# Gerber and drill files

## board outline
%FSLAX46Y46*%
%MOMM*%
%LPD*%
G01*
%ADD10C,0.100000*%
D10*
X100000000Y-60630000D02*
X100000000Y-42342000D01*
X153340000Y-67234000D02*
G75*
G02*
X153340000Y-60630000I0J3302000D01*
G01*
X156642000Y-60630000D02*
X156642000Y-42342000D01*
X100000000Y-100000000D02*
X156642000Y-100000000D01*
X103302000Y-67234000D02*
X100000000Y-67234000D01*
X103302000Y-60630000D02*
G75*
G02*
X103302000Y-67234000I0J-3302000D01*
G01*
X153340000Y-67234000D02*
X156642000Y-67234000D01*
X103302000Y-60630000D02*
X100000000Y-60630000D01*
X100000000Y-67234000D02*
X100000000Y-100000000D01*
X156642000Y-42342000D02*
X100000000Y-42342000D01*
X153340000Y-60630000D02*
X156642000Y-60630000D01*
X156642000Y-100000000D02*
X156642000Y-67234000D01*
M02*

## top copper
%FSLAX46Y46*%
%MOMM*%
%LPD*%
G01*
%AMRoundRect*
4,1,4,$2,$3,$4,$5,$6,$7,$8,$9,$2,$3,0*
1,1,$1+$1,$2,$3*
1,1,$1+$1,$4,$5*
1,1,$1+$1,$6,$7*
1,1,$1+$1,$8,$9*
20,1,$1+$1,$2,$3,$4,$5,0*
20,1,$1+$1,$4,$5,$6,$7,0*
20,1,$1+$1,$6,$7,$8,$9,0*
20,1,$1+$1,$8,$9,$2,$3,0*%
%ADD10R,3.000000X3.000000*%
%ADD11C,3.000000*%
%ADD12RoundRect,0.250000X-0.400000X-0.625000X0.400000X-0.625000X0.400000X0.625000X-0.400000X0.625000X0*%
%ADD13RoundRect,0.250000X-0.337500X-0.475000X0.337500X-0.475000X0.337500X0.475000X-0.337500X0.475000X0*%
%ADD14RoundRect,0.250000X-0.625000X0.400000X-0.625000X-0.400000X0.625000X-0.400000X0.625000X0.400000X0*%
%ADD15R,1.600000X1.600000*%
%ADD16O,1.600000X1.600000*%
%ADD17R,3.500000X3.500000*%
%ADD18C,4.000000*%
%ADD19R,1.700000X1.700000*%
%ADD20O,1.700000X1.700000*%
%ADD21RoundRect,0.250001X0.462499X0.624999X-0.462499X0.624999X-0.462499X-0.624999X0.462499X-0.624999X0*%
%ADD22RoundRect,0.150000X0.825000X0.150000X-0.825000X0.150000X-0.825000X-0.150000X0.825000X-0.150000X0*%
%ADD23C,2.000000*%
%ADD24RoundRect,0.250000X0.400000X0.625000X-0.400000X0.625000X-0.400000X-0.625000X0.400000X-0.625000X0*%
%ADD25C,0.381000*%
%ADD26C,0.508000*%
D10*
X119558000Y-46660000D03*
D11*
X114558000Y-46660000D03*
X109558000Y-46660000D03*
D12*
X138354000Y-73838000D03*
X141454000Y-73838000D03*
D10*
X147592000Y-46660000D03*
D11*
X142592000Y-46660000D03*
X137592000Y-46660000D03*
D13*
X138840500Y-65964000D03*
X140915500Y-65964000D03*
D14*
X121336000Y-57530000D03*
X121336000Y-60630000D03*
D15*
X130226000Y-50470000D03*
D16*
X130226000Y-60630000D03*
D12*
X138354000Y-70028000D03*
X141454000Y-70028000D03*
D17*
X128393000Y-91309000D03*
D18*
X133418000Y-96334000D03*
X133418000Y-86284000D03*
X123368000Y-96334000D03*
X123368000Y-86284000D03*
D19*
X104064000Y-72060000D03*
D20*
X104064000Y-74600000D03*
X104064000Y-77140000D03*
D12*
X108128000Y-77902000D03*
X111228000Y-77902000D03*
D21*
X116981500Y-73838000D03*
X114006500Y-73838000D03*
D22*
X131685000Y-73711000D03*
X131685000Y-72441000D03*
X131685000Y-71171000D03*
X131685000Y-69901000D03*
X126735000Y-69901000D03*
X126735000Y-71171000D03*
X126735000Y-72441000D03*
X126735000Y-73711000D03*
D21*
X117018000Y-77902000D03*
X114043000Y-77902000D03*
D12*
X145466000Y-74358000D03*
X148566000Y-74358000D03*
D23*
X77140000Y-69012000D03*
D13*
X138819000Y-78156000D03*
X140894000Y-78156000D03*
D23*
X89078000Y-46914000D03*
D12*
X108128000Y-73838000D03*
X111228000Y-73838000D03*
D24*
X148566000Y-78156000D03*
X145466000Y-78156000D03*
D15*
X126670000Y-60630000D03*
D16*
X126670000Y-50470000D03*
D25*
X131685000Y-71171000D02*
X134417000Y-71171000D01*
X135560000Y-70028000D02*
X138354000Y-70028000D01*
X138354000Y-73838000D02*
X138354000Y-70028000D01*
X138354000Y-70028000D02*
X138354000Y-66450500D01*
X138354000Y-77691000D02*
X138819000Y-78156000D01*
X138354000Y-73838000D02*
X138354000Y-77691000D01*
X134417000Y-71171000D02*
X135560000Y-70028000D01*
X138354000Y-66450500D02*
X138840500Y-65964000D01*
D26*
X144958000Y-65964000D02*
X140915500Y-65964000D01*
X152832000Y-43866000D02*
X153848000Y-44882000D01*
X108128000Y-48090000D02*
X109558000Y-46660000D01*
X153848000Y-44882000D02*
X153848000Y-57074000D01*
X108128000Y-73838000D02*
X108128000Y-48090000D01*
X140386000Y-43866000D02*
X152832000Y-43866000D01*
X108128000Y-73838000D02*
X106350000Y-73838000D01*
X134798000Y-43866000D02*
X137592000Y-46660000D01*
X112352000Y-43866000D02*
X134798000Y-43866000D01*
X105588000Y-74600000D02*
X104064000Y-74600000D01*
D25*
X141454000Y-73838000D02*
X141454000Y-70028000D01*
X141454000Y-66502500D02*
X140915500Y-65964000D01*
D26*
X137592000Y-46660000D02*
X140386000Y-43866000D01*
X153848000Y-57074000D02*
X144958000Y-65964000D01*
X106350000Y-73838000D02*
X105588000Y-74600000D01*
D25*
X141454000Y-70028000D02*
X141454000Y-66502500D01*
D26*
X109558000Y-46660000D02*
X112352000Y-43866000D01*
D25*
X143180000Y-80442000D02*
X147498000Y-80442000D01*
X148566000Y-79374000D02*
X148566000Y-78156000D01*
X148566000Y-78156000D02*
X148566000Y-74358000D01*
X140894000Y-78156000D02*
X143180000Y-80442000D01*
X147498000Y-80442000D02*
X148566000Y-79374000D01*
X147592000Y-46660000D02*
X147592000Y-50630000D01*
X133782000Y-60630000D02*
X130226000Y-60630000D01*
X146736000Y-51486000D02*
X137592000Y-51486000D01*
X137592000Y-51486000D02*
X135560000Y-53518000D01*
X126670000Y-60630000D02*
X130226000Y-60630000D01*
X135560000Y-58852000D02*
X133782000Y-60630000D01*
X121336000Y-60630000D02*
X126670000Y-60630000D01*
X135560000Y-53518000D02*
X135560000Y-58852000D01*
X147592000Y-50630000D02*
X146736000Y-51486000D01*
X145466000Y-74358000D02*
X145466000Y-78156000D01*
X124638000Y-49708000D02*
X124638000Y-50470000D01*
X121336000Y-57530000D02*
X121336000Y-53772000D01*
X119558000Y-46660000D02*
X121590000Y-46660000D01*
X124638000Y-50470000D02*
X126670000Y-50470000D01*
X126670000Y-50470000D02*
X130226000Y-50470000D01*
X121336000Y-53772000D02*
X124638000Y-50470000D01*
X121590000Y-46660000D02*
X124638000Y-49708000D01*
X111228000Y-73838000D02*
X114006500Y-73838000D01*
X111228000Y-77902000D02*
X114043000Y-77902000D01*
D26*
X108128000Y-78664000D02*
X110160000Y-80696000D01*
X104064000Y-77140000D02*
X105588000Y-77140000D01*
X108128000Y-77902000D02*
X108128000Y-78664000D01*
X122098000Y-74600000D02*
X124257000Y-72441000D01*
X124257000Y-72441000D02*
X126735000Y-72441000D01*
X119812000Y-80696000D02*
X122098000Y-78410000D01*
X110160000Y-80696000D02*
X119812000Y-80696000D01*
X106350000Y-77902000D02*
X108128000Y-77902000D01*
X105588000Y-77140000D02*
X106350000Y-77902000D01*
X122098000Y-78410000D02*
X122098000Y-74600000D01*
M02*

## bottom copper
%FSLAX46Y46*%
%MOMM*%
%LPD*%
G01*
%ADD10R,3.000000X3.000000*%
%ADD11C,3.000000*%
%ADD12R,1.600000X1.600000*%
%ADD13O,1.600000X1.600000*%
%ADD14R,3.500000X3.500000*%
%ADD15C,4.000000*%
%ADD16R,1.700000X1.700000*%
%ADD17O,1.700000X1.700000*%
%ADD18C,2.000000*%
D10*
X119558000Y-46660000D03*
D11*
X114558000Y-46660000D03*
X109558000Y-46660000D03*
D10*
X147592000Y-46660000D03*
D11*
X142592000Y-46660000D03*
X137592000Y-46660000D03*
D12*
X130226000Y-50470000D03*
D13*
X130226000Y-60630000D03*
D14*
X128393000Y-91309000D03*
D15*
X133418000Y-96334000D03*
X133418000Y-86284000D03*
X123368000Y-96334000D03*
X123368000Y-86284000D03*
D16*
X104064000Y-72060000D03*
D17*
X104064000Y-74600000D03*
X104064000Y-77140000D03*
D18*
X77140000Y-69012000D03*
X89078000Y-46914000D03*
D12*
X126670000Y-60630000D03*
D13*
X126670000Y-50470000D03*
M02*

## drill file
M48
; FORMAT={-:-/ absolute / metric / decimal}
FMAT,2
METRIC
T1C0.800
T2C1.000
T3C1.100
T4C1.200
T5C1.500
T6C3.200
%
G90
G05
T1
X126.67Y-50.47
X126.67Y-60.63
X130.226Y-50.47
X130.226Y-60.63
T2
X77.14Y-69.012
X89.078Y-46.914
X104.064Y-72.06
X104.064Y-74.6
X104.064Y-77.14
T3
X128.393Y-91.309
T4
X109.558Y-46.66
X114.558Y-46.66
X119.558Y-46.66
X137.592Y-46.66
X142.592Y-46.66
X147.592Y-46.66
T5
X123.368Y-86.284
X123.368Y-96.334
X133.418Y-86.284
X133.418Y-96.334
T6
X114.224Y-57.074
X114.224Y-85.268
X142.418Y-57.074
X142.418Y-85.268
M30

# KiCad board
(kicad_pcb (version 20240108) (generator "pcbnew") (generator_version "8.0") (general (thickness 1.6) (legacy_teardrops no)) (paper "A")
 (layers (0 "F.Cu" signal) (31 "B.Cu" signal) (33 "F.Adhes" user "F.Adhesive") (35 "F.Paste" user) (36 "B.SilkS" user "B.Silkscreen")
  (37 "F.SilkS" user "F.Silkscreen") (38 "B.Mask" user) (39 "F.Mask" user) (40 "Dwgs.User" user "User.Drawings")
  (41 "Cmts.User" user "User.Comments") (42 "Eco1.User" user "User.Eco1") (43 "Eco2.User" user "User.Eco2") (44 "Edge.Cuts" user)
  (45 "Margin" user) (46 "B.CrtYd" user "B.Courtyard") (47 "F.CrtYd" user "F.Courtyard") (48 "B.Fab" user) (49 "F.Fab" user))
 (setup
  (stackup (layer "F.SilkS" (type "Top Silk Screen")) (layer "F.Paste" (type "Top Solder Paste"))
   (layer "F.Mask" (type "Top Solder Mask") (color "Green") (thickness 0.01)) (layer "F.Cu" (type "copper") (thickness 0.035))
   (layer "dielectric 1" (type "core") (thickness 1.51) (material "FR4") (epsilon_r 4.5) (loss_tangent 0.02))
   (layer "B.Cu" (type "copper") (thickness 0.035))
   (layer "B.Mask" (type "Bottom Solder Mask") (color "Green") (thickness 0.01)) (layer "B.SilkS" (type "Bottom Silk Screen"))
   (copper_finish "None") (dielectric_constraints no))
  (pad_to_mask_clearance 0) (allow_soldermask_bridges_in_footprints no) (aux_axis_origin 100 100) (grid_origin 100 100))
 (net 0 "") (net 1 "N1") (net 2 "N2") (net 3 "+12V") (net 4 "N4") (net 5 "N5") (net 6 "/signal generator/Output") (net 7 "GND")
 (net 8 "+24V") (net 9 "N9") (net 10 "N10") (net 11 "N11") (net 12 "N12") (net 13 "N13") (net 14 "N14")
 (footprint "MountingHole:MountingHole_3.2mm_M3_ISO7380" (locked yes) (layer "F.Cu") (at 142.418 85.268)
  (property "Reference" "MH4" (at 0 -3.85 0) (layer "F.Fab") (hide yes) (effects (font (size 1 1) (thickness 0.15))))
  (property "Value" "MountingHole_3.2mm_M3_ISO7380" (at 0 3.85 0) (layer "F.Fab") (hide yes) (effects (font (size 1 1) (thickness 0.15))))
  (pad "" np_thru_hole circle (at 0 0) (size 3.2 3.2) (drill 3.2) (layers "*.Cu" "*.Mask")))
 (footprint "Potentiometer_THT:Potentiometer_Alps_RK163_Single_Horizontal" (layer "F.Cu") (at 119.558 46.66 -90)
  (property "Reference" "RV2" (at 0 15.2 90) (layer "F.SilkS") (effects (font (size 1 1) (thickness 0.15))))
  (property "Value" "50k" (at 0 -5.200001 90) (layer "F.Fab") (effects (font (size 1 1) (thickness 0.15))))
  (pad "1" thru_hole rect (at 0 0 90) (size 3 3) (drill 1.2) (layers "*.Cu" "*.Mask") (remove_unused_layers no) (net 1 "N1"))
  (pad "2" thru_hole circle (at 0 5 90) (size 3 3) (drill 1.2) (layers "*.Cu" "*.Mask") (remove_unused_layers no) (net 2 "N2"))
  (pad "3" thru_hole circle (at 0 10 90) (size 3 3) (drill 1.2) (layers "*.Cu" "*.Mask") (remove_unused_layers no) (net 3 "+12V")))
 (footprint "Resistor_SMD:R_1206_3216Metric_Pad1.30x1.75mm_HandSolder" (layer "F.Cu") (at 139.904 73.838)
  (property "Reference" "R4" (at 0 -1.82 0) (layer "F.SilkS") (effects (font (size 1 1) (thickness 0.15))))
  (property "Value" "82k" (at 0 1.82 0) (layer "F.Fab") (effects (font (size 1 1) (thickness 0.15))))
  (pad "1" smd roundrect (at -1.55 0) (size 1.3 1.75) (layers "F.Cu" "F.Paste" "F.Mask") (roundrect_rratio 0.192308) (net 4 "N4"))
  (pad "2" smd roundrect (at 1.55 0) (size 1.3 1.75) (layers "F.Cu" "F.Paste" "F.Mask") (roundrect_rratio 0.192308) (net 3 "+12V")))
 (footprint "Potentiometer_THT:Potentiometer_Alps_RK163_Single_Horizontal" (layer "F.Cu") (at 147.592 46.66 -90)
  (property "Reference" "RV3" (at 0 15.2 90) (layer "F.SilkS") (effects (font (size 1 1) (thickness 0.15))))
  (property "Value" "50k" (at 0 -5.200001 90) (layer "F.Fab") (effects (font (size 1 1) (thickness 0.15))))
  (pad "1" thru_hole rect (at 0 0 90) (size 3 3) (drill 1.2) (layers "*.Cu" "*.Mask") (remove_unused_layers no) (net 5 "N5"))
  (pad "2" thru_hole circle (at 0 5 90) (size 3 3) (drill 1.2) (layers "*.Cu" "*.Mask") (remove_unused_layers no)
   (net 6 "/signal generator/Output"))
  (pad "3" thru_hole circle (at 0 10 90) (size 3 3) (drill 1.2) (layers "*.Cu" "*.Mask") (remove_unused_layers no) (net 3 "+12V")))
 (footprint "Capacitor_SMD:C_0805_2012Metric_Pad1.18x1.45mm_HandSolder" (layer "F.Cu") (at 139.878 65.964)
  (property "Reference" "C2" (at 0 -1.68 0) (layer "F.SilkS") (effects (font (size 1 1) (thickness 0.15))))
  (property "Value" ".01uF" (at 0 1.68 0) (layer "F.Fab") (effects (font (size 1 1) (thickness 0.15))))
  (pad "1" smd roundrect (at -1.0375 0) (size 1.175 1.45) (layers "F.Cu" "F.Paste" "F.Mask") (roundrect_rratio 0.212766) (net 4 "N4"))
  (pad "2" smd roundrect (at 1.0375 0) (size 1.175 1.45) (layers "F.Cu" "F.Paste" "F.Mask") (roundrect_rratio 0.212766) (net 3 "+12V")))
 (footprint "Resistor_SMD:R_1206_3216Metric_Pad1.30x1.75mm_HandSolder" (layer "F.Cu") (at 121.336 59.08 -90)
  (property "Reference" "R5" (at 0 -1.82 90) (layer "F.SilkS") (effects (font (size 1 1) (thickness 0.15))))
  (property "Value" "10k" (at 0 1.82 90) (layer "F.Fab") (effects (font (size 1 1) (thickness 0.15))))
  (pad "1" smd roundrect (at -1.55 0 270) (size 1.3 1.75) (layers "F.Cu" "F.Paste" "F.Mask") (roundrect_rratio 0.192308) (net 1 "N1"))
  (pad "2" smd roundrect (at 1.55 0 270) (size 1.3 1.75) (layers "F.Cu" "F.Paste" "F.Mask") (roundrect_rratio 0.192308) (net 5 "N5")))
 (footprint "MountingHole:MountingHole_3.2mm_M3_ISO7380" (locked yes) (layer "F.Cu") (at 114.224 85.268)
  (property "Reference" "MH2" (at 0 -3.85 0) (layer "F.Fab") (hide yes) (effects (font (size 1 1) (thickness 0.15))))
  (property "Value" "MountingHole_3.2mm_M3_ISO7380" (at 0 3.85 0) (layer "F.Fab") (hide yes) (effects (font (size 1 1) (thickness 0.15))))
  (pad "" np_thru_hole circle (at 0 0) (size 3.2 3.2) (drill 3.2) (layers "*.Cu" "*.Mask")))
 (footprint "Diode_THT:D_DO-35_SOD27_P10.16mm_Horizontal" (layer "F.Cu") (at 130.226 50.47 -90)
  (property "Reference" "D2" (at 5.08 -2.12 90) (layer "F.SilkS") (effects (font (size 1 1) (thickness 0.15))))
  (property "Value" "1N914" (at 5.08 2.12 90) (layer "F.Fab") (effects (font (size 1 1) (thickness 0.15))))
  (pad "1" thru_hole rect (at 0 0 270) (size 1.6 1.6) (drill 0.8) (layers "*.Cu" "*.Mask") (remove_unused_layers no) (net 1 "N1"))
  (pad "2" thru_hole oval (at 10.16 0 270) (size 1.6 1.6) (drill 0.8) (layers "*.Cu" "*.Mask") (remove_unused_layers no) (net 5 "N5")))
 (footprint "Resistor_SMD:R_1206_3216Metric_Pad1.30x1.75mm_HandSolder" (layer "F.Cu") (at 139.904 70.028)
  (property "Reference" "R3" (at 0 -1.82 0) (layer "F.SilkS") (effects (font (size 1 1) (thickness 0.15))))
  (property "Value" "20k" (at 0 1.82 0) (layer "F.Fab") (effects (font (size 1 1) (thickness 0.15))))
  (pad "1" smd roundrect (at -1.55 0) (size 1.3 1.75) (layers "F.Cu" "F.Paste" "F.Mask") (roundrect_rratio 0.192308) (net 4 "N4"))
  (pad "2" smd roundrect (at 1.55 0) (size 1.3 1.75) (layers "F.Cu" "F.Paste" "F.Mask") (roundrect_rratio 0.192308) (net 3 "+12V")))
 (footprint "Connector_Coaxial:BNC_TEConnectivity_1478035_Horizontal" (layer "F.Cu") (at 128.393 91.309 180)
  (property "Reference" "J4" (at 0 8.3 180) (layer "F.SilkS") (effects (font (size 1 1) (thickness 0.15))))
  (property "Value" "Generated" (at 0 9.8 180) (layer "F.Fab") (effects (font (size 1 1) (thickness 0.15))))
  (pad "1" thru_hole rect (at 0 0 180) (size 3.5 3.5) (drill 1.1) (layers "*.Cu" "*.Mask") (remove_unused_layers no)
   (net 6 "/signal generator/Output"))
  (pad "2" thru_hole circle (at -5.025 -5.025 180) (size 4 4) (drill 1.5) (layers "*.Cu" "*.Mask") (remove_unused_layers no) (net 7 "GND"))
  (pad "2" thru_hole circle (at -5.025 5.025 180) (size 4 4) (drill 1.5) (layers "*.Cu" "*.Mask") (remove_unused_layers no) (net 7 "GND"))
  (pad "2" thru_hole circle (at 5.025 -5.025 180) (size 4 4) (drill 1.5) (layers "*.Cu" "*.Mask") (remove_unused_layers no) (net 7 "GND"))
  (pad "2" thru_hole circle (at 5.025 5.025 180) (size 4 4) (drill 1.5) (layers "*.Cu" "*.Mask") (remove_unused_layers no) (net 7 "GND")))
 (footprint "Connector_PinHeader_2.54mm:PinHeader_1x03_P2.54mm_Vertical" (layer "F.Cu") (at 104.064 72.06)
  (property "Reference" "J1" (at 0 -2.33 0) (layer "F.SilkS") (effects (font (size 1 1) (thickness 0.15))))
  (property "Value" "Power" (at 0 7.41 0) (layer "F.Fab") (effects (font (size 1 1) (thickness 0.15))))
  (pad "1" thru_hole rect (at 0 0) (size 1.7 1.7) (drill 1) (layers "*.Cu" "*.Mask") (remove_unused_layers no) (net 7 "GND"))
  (pad "2" thru_hole oval (at 0 2.54) (size 1.7 1.7) (drill 1) (layers "*.Cu" "*.Mask") (remove_unused_layers no) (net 3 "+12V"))
  (pad "3" thru_hole oval (at 0 5.08) (size 1.7 1.7) (drill 1) (layers "*.Cu" "*.Mask") (remove_unused_layers no) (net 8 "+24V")))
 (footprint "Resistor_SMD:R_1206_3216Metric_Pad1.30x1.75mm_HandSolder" (layer "F.Cu") (at 109.678 77.902)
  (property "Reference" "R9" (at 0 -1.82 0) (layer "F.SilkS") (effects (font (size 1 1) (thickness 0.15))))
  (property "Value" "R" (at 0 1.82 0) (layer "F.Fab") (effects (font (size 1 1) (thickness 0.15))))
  (pad "1" smd roundrect (at -1.55 0) (size 1.3 1.75) (layers "F.Cu" "F.Paste" "F.Mask") (roundrect_rratio 0.192308) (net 8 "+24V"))
  (pad "2" smd roundrect (at 1.55 0) (size 1.3 1.75) (layers "F.Cu" "F.Paste" "F.Mask") (roundrect_rratio 0.192308) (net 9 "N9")))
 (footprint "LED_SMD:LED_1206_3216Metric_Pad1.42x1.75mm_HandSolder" (layer "F.Cu") (at 115.494 73.838 180)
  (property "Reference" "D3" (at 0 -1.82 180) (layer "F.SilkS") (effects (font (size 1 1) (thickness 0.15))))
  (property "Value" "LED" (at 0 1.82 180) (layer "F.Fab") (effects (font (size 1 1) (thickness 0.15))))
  (pad "1" smd roundrect (at -1.4875 0 180) (size 1.425 1.75) (layers "F.Cu" "F.Paste" "F.Mask") (roundrect_rratio 0.175439) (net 7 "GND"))
  (pad "2" smd roundrect (at 1.4875 0 180) (size 1.425 1.75) (layers "F.Cu" "F.Paste" "F.Mask") (roundrect_rratio 0.175439) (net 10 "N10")))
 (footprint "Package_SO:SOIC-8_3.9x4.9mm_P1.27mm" (layer "F.Cu") (at 129.21 71.806 180)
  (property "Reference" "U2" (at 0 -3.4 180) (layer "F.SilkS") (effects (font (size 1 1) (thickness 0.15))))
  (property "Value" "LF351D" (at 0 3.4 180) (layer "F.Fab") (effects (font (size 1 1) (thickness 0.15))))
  (pad "1" smd roundrect (at -2.475 -1.905 180) (size 1.95 0.6) (layers "F.Cu" "F.Paste" "F.Mask") (roundrect_rratio 0.25) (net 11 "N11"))
  (pad "2" smd roundrect (at -2.475 -0.635 180) (size 1.95 0.6) (layers "F.Cu" "F.Paste" "F.Mask") (roundrect_rratio 0.25) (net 2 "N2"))
  (pad "3" smd roundrect (at -2.475 0.635 180) (size 1.95 0.6) (layers "F.Cu" "F.Paste" "F.Mask") (roundrect_rratio 0.25) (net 4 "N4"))
  (pad "4" smd roundrect (at -2.475 1.905 180) (size 1.95 0.6) (layers "F.Cu" "F.Paste" "F.Mask") (roundrect_rratio 0.25) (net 7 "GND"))
  (pad "5" smd roundrect (at 2.475 1.905 180) (size 1.95 0.6) (layers "F.Cu" "F.Paste" "F.Mask") (roundrect_rratio 0.25) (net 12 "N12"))
  (pad "6" smd roundrect (at 2.475 0.635 180) (size 1.95 0.6) (layers "F.Cu" "F.Paste" "F.Mask") (roundrect_rratio 0.25) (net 5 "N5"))
  (pad "7" smd roundrect (at 2.475 -0.635 180) (size 1.95 0.6) (layers "F.Cu" "F.Paste" "F.Mask") (roundrect_rratio 0.25) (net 8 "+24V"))
  (pad "8" smd roundrect (at 2.475 -1.905 180) (size 1.95 0.6) (layers "F.Cu" "F.Paste" "F.Mask") (roundrect_rratio 0.25) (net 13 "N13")))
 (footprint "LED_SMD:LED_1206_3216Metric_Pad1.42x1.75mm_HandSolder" (layer "F.Cu") (at 115.5305 77.902 180)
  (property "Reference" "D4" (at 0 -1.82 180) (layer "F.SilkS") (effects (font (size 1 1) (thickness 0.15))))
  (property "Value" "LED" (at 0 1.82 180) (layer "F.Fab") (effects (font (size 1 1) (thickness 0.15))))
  (pad "1" smd roundrect (at -1.4875 0 180) (size 1.425 1.75) (layers "F.Cu" "F.Paste" "F.Mask") (roundrect_rratio 0.175439) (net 7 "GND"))
  (pad "2" smd roundrect (at 1.4875 0 180) (size 1.425 1.75) (layers "F.Cu" "F.Paste" "F.Mask") (roundrect_rratio 0.175439) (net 9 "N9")))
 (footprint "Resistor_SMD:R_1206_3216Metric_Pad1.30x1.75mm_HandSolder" (layer "F.Cu") (at 147.016 74.358)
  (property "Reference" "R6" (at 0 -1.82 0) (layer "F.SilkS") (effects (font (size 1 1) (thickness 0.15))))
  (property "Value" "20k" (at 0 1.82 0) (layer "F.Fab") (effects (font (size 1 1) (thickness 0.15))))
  (pad "1" smd roundrect (at -1.55 0) (size 1.3 1.75) (layers "F.Cu" "F.Paste" "F.Mask") (roundrect_rratio 0.192308) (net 5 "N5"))
  (pad "2" smd roundrect (at 1.55 0) (size 1.3 1.75) (layers "F.Cu" "F.Paste" "F.Mask") (roundrect_rratio 0.192308) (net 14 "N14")))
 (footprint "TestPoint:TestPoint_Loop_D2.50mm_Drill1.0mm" (layer "F.Cu") (at 77.14 69.012)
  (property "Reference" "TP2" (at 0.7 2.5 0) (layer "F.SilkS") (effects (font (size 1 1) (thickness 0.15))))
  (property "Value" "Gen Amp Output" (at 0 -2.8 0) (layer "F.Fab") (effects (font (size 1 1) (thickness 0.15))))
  (pad "1" thru_hole circle (at 0 0) (size 2 2) (drill 1) (layers "*.Cu" "*.Mask") (remove_unused_layers no) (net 5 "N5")))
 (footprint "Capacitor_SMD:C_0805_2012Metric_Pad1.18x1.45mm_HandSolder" (layer "F.Cu") (at 139.8565 78.156)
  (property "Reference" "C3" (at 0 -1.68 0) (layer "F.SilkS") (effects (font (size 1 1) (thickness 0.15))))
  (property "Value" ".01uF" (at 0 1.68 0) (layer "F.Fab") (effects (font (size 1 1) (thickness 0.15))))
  (pad "1" smd roundrect (at -1.0375 0) (size 1.175 1.45) (layers "F.Cu" "F.Paste" "F.Mask") (roundrect_rratio 0.212766) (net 4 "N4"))
  (pad "2" smd roundrect (at 1.0375 0) (size 1.175 1.45) (layers "F.Cu" "F.Paste" "F.Mask") (roundrect_rratio 0.212766) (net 14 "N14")))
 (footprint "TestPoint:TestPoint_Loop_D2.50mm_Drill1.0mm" (layer "F.Cu") (at 89.078 46.914)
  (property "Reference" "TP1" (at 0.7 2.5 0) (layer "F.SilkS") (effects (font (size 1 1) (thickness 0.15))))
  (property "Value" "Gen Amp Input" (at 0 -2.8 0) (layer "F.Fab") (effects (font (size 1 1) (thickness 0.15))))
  (pad "1" thru_hole circle (at 0 0) (size 2 2) (drill 1) (layers "*.Cu" "*.Mask") (remove_unused_layers no) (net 2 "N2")))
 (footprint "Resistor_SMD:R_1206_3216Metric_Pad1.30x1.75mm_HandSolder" (layer "F.Cu") (at 109.678 73.838)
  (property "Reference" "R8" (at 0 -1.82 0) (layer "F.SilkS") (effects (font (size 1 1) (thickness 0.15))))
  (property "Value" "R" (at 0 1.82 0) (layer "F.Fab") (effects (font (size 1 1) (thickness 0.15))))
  (pad "1" smd roundrect (at -1.55 0) (size 1.3 1.75) (layers "F.Cu" "F.Paste" "F.Mask") (roundrect_rratio 0.192308) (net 3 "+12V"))
  (pad "2" smd roundrect (at 1.55 0) (size 1.3 1.75) (layers "F.Cu" "F.Paste" "F.Mask") (roundrect_rratio 0.192308) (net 10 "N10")))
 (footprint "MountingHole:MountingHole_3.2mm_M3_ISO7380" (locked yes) (layer "F.Cu") (at 142.418 57.074)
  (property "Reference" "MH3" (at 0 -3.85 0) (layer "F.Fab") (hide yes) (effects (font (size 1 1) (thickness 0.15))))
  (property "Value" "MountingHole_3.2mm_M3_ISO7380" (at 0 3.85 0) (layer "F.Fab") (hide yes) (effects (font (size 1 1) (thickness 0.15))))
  (pad "" np_thru_hole circle (at 0 0) (size 3.2 3.2) (drill 3.2) (layers "*.Cu" "*.Mask")))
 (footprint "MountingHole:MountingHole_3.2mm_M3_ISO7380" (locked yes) (layer "F.Cu") (at 114.224 57.074)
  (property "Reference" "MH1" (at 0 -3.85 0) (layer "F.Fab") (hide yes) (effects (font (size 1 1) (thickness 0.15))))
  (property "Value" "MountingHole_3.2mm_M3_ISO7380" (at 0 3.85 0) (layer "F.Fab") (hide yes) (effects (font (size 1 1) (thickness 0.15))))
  (pad "" np_thru_hole circle (at 0 0) (size 3.2 3.2) (drill 3.2) (layers "*.Cu" "*.Mask")))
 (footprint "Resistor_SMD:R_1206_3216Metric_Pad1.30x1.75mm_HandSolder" (layer "F.Cu") (at 147.016 78.156 180)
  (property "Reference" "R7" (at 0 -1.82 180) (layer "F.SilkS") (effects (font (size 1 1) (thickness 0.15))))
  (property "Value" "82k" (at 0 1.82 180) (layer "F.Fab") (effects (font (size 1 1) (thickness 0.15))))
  (pad "1" smd roundrect (at -1.55 0 180) (size 1.3 1.75) (layers "F.Cu" "F.Paste" "F.Mask") (roundrect_rratio 0.192308) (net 14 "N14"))
  (pad "2" smd roundrect (at 1.55 0 180) (size 1.3 1.75) (layers "F.Cu" "F.Paste" "F.Mask") (roundrect_rratio 0.192308) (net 5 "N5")))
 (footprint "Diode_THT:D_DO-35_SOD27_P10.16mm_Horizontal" (layer "F.Cu") (at 126.67 60.63 90)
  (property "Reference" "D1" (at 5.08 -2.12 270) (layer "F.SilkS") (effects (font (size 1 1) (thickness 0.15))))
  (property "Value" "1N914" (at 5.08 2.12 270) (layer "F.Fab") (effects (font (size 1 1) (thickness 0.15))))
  (pad "1" thru_hole rect (at 0 0 90) (size 1.6 1.6) (drill 0.8) (layers "*.Cu" "*.Mask") (remove_unused_layers no) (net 5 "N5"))
  (pad "2" thru_hole oval (at 10.16 0 90) (size 1.6 1.6) (drill 0.8) (layers "*.Cu" "*.Mask") (remove_unused_layers no) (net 1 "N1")))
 (gr_line (start 100 60.63) (end 100 42.342) (locked yes) (stroke (width 0.1) (type solid)) (layer "Edge.Cuts"))
 (gr_arc (start 153.34 67.234) (mid 150.038 63.932) (end 153.34 60.63) (locked yes) (stroke (width 0.1) (type solid)) (layer "Edge.Cuts"))
 (gr_line (start 156.642 60.63) (end 156.642 42.342) (locked yes) (stroke (width 0.1) (type solid)) (layer "Edge.Cuts"))
 (gr_line (start 100 100) (end 156.642 100) (locked yes) (stroke (width 0.1) (type solid)) (layer "Edge.Cuts"))
 (gr_line (start 103.302 67.234) (end 100 67.234) (locked yes) (stroke (width 0.1) (type solid)) (layer "Edge.Cuts"))
 (gr_arc (start 103.302 60.63) (mid 106.604 63.932) (end 103.302 67.234) (locked yes) (stroke (width 0.1) (type solid)) (layer "Edge.Cuts"))
 (gr_line (start 153.34 67.234) (end 156.642 67.234) (locked yes) (stroke (width 0.1) (type solid)) (layer "Edge.Cuts"))
 (gr_line (start 103.302 60.63) (end 100 60.63) (locked yes) (stroke (width 0.1) (type solid)) (layer "Edge.Cuts"))
 (gr_line (start 100 67.234) (end 100 100) (locked yes) (stroke (width 0.1) (type solid)) (layer "Edge.Cuts"))
 (gr_line (start 156.642 42.342) (end 100 42.342) (locked yes) (stroke (width 0.1) (type solid)) (layer "Edge.Cuts"))
 (gr_line (start 153.34 60.63) (end 156.642 60.63) (locked yes) (stroke (width 0.1) (type solid)) (layer "Edge.Cuts"))
 (gr_line (start 156.642 100) (end 156.642 67.234) (locked yes) (stroke (width 0.1) (type solid)) (layer "Edge.Cuts"))
 (segment (start 131.685 71.171) (end 134.417 71.171) (width 0.381) (layer "F.Cu") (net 4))
 (segment (start 135.56 70.028) (end 138.354 70.028) (width 0.381) (layer "F.Cu") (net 4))
 (segment (start 138.354 73.838) (end 138.354 70.028) (width 0.381) (layer "F.Cu") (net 4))
 (segment (start 138.354 70.028) (end 138.354 66.4505) (width 0.381) (layer "F.Cu") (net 4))
 (segment (start 138.354 77.691) (end 138.819 78.156) (width 0.381) (layer "F.Cu") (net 4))
 (segment (start 138.354 73.838) (end 138.354 77.691) (width 0.381) (layer "F.Cu") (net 4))
 (segment (start 134.417 71.171) (end 135.56 70.028) (width 0.381) (layer "F.Cu") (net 4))
 (segment (start 138.354 66.4505) (end 138.8405 65.964) (width 0.381) (layer "F.Cu") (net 4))
 (segment (start 144.958 65.964) (end 140.9155 65.964) (width 0.508) (layer "F.Cu") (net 3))
 (segment (start 152.832 43.866) (end 153.848 44.882) (width 0.508) (layer "F.Cu") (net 3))
 (segment (start 108.128 48.09) (end 109.558 46.66) (width 0.508) (layer "F.Cu") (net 3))
 (segment (start 153.848 44.882) (end 153.848 57.074) (width 0.508) (layer "F.Cu") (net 3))
 (segment (start 108.128 73.838) (end 108.128 48.09) (width 0.508) (layer "F.Cu") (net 3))
 (segment (start 140.386 43.866) (end 152.832 43.866) (width 0.508) (layer "F.Cu") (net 3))
 (segment (start 108.128 73.838) (end 106.35 73.838) (width 0.508) (layer "F.Cu") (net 3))
 (segment (start 134.798 43.866) (end 137.592 46.66) (width 0.508) (layer "F.Cu") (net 3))
 (segment (start 112.352 43.866) (end 134.798 43.866) (width 0.508) (layer "F.Cu") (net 3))
 (segment (start 105.588 74.6) (end 104.064 74.6) (width 0.508) (layer "F.Cu") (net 3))
 (segment (start 141.454 73.838) (end 141.454 70.028) (width 0.381) (layer "F.Cu") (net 3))
 (segment (start 141.454 66.5025) (end 140.9155 65.964) (width 0.381) (layer "F.Cu") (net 3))
 (segment (start 137.592 46.66) (end 140.386 43.866) (width 0.508) (layer "F.Cu") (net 3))
 (segment (start 153.848 57.074) (end 144.958 65.964) (width 0.508) (layer "F.Cu") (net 3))
 (segment (start 106.35 73.838) (end 105.588 74.6) (width 0.508) (layer "F.Cu") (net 3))
 (segment (start 141.454 70.028) (end 141.454 66.5025) (width 0.381) (layer "F.Cu") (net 3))
 (segment (start 109.558 46.66) (end 112.352 43.866) (width 0.508) (layer "F.Cu") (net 3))
 (segment (start 143.18 80.442) (end 147.498 80.442) (width 0.381) (layer "F.Cu") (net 14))
 (segment (start 148.566 79.374) (end 148.566 78.156) (width 0.381) (layer "F.Cu") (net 14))
 (segment (start 148.566 78.156) (end 148.566 74.358) (width 0.381) (layer "F.Cu") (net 14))
 (segment (start 140.894 78.156) (end 143.18 80.442) (width 0.381) (layer "F.Cu") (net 14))
 (segment (start 147.498 80.442) (end 148.566 79.374) (width 0.381) (layer "F.Cu") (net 14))
 (segment (start 147.592 46.66) (end 147.592 50.63) (width 0.381) (layer "F.Cu") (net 5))
 (segment (start 133.782 60.63) (end 130.226 60.63) (width 0.381) (layer "F.Cu") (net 5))
 (segment (start 146.736 51.486) (end 137.592 51.486) (width 0.381) (layer "F.Cu") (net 5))
 (segment (start 137.592 51.486) (end 135.56 53.518) (width 0.381) (layer "F.Cu") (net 5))
 (segment (start 126.67 60.63) (end 130.226 60.63) (width 0.381) (layer "F.Cu") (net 5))
 (segment (start 135.56 58.852) (end 133.782 60.63) (width 0.381) (layer "F.Cu") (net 5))
 (segment (start 121.336 60.63) (end 126.67 60.63) (width 0.381) (layer "F.Cu") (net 5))
 (segment (start 135.56 53.518) (end 135.56 58.852) (width 0.381) (layer "F.Cu") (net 5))
 (segment (start 147.592 50.63) (end 146.736 51.486) (width 0.381) (layer "F.Cu") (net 5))
 (segment (start 145.466 74.358) (end 145.466 78.156) (width 0.381) (layer "F.Cu") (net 5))
 (segment (start 124.638 49.708) (end 124.638 50.47) (width 0.381) (layer "F.Cu") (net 1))
 (segment (start 121.336 57.53) (end 121.336 53.772) (width 0.381) (layer "F.Cu") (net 1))
 (segment (start 119.558 46.66) (end 121.59 46.66) (width 0.381) (layer "F.Cu") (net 1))
 (segment (start 124.638 50.47) (end 126.67 50.47) (width 0.381) (layer "F.Cu") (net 1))
 (segment (start 126.67 50.47) (end 130.226 50.47) (width 0.381) (layer "F.Cu") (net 1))
 (segment (start 121.336 53.772) (end 124.638 50.47) (width 0.381) (layer "F.Cu") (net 1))
 (segment (start 121.59 46.66) (end 124.638 49.708) (width 0.381) (layer "F.Cu") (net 1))
 (segment (start 111.228 73.838) (end 114.0065 73.838) (width 0.381) (layer "F.Cu") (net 10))
 (segment (start 111.228 77.902) (end 114.043 77.902) (width 0.381) (layer "F.Cu") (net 9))
 (segment (start 108.128 78.664) (end 110.16 80.696) (width 0.508) (layer "F.Cu") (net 8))
 (segment (start 104.064 77.14) (end 105.588 77.14) (width 0.508) (layer "F.Cu") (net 8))
 (segment (start 108.128 77.902) (end 108.128 78.664) (width 0.508) (layer "F.Cu") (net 8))
 (segment (start 122.098 74.6) (end 124.257 72.441) (width 0.508) (layer "F.Cu") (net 8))
 (segment (start 124.257 72.441) (end 126.735 72.441) (width 0.508) (layer "F.Cu") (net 8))
 (segment (start 119.812 80.696) (end 122.098 78.41) (width 0.508) (layer "F.Cu") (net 8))
 (segment (start 110.16 80.696) (end 119.812 80.696) (width 0.508) (layer "F.Cu") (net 8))
 (segment (start 106.35 77.902) (end 108.128 77.902) (width 0.508) (layer "F.Cu") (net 8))
 (segment (start 105.588 77.14) (end 106.35 77.902) (width 0.508) (layer "F.Cu") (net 8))
 (segment (start 122.098 78.41) (end 122.098 74.6) (width 0.508) (layer "F.Cu") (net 8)))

